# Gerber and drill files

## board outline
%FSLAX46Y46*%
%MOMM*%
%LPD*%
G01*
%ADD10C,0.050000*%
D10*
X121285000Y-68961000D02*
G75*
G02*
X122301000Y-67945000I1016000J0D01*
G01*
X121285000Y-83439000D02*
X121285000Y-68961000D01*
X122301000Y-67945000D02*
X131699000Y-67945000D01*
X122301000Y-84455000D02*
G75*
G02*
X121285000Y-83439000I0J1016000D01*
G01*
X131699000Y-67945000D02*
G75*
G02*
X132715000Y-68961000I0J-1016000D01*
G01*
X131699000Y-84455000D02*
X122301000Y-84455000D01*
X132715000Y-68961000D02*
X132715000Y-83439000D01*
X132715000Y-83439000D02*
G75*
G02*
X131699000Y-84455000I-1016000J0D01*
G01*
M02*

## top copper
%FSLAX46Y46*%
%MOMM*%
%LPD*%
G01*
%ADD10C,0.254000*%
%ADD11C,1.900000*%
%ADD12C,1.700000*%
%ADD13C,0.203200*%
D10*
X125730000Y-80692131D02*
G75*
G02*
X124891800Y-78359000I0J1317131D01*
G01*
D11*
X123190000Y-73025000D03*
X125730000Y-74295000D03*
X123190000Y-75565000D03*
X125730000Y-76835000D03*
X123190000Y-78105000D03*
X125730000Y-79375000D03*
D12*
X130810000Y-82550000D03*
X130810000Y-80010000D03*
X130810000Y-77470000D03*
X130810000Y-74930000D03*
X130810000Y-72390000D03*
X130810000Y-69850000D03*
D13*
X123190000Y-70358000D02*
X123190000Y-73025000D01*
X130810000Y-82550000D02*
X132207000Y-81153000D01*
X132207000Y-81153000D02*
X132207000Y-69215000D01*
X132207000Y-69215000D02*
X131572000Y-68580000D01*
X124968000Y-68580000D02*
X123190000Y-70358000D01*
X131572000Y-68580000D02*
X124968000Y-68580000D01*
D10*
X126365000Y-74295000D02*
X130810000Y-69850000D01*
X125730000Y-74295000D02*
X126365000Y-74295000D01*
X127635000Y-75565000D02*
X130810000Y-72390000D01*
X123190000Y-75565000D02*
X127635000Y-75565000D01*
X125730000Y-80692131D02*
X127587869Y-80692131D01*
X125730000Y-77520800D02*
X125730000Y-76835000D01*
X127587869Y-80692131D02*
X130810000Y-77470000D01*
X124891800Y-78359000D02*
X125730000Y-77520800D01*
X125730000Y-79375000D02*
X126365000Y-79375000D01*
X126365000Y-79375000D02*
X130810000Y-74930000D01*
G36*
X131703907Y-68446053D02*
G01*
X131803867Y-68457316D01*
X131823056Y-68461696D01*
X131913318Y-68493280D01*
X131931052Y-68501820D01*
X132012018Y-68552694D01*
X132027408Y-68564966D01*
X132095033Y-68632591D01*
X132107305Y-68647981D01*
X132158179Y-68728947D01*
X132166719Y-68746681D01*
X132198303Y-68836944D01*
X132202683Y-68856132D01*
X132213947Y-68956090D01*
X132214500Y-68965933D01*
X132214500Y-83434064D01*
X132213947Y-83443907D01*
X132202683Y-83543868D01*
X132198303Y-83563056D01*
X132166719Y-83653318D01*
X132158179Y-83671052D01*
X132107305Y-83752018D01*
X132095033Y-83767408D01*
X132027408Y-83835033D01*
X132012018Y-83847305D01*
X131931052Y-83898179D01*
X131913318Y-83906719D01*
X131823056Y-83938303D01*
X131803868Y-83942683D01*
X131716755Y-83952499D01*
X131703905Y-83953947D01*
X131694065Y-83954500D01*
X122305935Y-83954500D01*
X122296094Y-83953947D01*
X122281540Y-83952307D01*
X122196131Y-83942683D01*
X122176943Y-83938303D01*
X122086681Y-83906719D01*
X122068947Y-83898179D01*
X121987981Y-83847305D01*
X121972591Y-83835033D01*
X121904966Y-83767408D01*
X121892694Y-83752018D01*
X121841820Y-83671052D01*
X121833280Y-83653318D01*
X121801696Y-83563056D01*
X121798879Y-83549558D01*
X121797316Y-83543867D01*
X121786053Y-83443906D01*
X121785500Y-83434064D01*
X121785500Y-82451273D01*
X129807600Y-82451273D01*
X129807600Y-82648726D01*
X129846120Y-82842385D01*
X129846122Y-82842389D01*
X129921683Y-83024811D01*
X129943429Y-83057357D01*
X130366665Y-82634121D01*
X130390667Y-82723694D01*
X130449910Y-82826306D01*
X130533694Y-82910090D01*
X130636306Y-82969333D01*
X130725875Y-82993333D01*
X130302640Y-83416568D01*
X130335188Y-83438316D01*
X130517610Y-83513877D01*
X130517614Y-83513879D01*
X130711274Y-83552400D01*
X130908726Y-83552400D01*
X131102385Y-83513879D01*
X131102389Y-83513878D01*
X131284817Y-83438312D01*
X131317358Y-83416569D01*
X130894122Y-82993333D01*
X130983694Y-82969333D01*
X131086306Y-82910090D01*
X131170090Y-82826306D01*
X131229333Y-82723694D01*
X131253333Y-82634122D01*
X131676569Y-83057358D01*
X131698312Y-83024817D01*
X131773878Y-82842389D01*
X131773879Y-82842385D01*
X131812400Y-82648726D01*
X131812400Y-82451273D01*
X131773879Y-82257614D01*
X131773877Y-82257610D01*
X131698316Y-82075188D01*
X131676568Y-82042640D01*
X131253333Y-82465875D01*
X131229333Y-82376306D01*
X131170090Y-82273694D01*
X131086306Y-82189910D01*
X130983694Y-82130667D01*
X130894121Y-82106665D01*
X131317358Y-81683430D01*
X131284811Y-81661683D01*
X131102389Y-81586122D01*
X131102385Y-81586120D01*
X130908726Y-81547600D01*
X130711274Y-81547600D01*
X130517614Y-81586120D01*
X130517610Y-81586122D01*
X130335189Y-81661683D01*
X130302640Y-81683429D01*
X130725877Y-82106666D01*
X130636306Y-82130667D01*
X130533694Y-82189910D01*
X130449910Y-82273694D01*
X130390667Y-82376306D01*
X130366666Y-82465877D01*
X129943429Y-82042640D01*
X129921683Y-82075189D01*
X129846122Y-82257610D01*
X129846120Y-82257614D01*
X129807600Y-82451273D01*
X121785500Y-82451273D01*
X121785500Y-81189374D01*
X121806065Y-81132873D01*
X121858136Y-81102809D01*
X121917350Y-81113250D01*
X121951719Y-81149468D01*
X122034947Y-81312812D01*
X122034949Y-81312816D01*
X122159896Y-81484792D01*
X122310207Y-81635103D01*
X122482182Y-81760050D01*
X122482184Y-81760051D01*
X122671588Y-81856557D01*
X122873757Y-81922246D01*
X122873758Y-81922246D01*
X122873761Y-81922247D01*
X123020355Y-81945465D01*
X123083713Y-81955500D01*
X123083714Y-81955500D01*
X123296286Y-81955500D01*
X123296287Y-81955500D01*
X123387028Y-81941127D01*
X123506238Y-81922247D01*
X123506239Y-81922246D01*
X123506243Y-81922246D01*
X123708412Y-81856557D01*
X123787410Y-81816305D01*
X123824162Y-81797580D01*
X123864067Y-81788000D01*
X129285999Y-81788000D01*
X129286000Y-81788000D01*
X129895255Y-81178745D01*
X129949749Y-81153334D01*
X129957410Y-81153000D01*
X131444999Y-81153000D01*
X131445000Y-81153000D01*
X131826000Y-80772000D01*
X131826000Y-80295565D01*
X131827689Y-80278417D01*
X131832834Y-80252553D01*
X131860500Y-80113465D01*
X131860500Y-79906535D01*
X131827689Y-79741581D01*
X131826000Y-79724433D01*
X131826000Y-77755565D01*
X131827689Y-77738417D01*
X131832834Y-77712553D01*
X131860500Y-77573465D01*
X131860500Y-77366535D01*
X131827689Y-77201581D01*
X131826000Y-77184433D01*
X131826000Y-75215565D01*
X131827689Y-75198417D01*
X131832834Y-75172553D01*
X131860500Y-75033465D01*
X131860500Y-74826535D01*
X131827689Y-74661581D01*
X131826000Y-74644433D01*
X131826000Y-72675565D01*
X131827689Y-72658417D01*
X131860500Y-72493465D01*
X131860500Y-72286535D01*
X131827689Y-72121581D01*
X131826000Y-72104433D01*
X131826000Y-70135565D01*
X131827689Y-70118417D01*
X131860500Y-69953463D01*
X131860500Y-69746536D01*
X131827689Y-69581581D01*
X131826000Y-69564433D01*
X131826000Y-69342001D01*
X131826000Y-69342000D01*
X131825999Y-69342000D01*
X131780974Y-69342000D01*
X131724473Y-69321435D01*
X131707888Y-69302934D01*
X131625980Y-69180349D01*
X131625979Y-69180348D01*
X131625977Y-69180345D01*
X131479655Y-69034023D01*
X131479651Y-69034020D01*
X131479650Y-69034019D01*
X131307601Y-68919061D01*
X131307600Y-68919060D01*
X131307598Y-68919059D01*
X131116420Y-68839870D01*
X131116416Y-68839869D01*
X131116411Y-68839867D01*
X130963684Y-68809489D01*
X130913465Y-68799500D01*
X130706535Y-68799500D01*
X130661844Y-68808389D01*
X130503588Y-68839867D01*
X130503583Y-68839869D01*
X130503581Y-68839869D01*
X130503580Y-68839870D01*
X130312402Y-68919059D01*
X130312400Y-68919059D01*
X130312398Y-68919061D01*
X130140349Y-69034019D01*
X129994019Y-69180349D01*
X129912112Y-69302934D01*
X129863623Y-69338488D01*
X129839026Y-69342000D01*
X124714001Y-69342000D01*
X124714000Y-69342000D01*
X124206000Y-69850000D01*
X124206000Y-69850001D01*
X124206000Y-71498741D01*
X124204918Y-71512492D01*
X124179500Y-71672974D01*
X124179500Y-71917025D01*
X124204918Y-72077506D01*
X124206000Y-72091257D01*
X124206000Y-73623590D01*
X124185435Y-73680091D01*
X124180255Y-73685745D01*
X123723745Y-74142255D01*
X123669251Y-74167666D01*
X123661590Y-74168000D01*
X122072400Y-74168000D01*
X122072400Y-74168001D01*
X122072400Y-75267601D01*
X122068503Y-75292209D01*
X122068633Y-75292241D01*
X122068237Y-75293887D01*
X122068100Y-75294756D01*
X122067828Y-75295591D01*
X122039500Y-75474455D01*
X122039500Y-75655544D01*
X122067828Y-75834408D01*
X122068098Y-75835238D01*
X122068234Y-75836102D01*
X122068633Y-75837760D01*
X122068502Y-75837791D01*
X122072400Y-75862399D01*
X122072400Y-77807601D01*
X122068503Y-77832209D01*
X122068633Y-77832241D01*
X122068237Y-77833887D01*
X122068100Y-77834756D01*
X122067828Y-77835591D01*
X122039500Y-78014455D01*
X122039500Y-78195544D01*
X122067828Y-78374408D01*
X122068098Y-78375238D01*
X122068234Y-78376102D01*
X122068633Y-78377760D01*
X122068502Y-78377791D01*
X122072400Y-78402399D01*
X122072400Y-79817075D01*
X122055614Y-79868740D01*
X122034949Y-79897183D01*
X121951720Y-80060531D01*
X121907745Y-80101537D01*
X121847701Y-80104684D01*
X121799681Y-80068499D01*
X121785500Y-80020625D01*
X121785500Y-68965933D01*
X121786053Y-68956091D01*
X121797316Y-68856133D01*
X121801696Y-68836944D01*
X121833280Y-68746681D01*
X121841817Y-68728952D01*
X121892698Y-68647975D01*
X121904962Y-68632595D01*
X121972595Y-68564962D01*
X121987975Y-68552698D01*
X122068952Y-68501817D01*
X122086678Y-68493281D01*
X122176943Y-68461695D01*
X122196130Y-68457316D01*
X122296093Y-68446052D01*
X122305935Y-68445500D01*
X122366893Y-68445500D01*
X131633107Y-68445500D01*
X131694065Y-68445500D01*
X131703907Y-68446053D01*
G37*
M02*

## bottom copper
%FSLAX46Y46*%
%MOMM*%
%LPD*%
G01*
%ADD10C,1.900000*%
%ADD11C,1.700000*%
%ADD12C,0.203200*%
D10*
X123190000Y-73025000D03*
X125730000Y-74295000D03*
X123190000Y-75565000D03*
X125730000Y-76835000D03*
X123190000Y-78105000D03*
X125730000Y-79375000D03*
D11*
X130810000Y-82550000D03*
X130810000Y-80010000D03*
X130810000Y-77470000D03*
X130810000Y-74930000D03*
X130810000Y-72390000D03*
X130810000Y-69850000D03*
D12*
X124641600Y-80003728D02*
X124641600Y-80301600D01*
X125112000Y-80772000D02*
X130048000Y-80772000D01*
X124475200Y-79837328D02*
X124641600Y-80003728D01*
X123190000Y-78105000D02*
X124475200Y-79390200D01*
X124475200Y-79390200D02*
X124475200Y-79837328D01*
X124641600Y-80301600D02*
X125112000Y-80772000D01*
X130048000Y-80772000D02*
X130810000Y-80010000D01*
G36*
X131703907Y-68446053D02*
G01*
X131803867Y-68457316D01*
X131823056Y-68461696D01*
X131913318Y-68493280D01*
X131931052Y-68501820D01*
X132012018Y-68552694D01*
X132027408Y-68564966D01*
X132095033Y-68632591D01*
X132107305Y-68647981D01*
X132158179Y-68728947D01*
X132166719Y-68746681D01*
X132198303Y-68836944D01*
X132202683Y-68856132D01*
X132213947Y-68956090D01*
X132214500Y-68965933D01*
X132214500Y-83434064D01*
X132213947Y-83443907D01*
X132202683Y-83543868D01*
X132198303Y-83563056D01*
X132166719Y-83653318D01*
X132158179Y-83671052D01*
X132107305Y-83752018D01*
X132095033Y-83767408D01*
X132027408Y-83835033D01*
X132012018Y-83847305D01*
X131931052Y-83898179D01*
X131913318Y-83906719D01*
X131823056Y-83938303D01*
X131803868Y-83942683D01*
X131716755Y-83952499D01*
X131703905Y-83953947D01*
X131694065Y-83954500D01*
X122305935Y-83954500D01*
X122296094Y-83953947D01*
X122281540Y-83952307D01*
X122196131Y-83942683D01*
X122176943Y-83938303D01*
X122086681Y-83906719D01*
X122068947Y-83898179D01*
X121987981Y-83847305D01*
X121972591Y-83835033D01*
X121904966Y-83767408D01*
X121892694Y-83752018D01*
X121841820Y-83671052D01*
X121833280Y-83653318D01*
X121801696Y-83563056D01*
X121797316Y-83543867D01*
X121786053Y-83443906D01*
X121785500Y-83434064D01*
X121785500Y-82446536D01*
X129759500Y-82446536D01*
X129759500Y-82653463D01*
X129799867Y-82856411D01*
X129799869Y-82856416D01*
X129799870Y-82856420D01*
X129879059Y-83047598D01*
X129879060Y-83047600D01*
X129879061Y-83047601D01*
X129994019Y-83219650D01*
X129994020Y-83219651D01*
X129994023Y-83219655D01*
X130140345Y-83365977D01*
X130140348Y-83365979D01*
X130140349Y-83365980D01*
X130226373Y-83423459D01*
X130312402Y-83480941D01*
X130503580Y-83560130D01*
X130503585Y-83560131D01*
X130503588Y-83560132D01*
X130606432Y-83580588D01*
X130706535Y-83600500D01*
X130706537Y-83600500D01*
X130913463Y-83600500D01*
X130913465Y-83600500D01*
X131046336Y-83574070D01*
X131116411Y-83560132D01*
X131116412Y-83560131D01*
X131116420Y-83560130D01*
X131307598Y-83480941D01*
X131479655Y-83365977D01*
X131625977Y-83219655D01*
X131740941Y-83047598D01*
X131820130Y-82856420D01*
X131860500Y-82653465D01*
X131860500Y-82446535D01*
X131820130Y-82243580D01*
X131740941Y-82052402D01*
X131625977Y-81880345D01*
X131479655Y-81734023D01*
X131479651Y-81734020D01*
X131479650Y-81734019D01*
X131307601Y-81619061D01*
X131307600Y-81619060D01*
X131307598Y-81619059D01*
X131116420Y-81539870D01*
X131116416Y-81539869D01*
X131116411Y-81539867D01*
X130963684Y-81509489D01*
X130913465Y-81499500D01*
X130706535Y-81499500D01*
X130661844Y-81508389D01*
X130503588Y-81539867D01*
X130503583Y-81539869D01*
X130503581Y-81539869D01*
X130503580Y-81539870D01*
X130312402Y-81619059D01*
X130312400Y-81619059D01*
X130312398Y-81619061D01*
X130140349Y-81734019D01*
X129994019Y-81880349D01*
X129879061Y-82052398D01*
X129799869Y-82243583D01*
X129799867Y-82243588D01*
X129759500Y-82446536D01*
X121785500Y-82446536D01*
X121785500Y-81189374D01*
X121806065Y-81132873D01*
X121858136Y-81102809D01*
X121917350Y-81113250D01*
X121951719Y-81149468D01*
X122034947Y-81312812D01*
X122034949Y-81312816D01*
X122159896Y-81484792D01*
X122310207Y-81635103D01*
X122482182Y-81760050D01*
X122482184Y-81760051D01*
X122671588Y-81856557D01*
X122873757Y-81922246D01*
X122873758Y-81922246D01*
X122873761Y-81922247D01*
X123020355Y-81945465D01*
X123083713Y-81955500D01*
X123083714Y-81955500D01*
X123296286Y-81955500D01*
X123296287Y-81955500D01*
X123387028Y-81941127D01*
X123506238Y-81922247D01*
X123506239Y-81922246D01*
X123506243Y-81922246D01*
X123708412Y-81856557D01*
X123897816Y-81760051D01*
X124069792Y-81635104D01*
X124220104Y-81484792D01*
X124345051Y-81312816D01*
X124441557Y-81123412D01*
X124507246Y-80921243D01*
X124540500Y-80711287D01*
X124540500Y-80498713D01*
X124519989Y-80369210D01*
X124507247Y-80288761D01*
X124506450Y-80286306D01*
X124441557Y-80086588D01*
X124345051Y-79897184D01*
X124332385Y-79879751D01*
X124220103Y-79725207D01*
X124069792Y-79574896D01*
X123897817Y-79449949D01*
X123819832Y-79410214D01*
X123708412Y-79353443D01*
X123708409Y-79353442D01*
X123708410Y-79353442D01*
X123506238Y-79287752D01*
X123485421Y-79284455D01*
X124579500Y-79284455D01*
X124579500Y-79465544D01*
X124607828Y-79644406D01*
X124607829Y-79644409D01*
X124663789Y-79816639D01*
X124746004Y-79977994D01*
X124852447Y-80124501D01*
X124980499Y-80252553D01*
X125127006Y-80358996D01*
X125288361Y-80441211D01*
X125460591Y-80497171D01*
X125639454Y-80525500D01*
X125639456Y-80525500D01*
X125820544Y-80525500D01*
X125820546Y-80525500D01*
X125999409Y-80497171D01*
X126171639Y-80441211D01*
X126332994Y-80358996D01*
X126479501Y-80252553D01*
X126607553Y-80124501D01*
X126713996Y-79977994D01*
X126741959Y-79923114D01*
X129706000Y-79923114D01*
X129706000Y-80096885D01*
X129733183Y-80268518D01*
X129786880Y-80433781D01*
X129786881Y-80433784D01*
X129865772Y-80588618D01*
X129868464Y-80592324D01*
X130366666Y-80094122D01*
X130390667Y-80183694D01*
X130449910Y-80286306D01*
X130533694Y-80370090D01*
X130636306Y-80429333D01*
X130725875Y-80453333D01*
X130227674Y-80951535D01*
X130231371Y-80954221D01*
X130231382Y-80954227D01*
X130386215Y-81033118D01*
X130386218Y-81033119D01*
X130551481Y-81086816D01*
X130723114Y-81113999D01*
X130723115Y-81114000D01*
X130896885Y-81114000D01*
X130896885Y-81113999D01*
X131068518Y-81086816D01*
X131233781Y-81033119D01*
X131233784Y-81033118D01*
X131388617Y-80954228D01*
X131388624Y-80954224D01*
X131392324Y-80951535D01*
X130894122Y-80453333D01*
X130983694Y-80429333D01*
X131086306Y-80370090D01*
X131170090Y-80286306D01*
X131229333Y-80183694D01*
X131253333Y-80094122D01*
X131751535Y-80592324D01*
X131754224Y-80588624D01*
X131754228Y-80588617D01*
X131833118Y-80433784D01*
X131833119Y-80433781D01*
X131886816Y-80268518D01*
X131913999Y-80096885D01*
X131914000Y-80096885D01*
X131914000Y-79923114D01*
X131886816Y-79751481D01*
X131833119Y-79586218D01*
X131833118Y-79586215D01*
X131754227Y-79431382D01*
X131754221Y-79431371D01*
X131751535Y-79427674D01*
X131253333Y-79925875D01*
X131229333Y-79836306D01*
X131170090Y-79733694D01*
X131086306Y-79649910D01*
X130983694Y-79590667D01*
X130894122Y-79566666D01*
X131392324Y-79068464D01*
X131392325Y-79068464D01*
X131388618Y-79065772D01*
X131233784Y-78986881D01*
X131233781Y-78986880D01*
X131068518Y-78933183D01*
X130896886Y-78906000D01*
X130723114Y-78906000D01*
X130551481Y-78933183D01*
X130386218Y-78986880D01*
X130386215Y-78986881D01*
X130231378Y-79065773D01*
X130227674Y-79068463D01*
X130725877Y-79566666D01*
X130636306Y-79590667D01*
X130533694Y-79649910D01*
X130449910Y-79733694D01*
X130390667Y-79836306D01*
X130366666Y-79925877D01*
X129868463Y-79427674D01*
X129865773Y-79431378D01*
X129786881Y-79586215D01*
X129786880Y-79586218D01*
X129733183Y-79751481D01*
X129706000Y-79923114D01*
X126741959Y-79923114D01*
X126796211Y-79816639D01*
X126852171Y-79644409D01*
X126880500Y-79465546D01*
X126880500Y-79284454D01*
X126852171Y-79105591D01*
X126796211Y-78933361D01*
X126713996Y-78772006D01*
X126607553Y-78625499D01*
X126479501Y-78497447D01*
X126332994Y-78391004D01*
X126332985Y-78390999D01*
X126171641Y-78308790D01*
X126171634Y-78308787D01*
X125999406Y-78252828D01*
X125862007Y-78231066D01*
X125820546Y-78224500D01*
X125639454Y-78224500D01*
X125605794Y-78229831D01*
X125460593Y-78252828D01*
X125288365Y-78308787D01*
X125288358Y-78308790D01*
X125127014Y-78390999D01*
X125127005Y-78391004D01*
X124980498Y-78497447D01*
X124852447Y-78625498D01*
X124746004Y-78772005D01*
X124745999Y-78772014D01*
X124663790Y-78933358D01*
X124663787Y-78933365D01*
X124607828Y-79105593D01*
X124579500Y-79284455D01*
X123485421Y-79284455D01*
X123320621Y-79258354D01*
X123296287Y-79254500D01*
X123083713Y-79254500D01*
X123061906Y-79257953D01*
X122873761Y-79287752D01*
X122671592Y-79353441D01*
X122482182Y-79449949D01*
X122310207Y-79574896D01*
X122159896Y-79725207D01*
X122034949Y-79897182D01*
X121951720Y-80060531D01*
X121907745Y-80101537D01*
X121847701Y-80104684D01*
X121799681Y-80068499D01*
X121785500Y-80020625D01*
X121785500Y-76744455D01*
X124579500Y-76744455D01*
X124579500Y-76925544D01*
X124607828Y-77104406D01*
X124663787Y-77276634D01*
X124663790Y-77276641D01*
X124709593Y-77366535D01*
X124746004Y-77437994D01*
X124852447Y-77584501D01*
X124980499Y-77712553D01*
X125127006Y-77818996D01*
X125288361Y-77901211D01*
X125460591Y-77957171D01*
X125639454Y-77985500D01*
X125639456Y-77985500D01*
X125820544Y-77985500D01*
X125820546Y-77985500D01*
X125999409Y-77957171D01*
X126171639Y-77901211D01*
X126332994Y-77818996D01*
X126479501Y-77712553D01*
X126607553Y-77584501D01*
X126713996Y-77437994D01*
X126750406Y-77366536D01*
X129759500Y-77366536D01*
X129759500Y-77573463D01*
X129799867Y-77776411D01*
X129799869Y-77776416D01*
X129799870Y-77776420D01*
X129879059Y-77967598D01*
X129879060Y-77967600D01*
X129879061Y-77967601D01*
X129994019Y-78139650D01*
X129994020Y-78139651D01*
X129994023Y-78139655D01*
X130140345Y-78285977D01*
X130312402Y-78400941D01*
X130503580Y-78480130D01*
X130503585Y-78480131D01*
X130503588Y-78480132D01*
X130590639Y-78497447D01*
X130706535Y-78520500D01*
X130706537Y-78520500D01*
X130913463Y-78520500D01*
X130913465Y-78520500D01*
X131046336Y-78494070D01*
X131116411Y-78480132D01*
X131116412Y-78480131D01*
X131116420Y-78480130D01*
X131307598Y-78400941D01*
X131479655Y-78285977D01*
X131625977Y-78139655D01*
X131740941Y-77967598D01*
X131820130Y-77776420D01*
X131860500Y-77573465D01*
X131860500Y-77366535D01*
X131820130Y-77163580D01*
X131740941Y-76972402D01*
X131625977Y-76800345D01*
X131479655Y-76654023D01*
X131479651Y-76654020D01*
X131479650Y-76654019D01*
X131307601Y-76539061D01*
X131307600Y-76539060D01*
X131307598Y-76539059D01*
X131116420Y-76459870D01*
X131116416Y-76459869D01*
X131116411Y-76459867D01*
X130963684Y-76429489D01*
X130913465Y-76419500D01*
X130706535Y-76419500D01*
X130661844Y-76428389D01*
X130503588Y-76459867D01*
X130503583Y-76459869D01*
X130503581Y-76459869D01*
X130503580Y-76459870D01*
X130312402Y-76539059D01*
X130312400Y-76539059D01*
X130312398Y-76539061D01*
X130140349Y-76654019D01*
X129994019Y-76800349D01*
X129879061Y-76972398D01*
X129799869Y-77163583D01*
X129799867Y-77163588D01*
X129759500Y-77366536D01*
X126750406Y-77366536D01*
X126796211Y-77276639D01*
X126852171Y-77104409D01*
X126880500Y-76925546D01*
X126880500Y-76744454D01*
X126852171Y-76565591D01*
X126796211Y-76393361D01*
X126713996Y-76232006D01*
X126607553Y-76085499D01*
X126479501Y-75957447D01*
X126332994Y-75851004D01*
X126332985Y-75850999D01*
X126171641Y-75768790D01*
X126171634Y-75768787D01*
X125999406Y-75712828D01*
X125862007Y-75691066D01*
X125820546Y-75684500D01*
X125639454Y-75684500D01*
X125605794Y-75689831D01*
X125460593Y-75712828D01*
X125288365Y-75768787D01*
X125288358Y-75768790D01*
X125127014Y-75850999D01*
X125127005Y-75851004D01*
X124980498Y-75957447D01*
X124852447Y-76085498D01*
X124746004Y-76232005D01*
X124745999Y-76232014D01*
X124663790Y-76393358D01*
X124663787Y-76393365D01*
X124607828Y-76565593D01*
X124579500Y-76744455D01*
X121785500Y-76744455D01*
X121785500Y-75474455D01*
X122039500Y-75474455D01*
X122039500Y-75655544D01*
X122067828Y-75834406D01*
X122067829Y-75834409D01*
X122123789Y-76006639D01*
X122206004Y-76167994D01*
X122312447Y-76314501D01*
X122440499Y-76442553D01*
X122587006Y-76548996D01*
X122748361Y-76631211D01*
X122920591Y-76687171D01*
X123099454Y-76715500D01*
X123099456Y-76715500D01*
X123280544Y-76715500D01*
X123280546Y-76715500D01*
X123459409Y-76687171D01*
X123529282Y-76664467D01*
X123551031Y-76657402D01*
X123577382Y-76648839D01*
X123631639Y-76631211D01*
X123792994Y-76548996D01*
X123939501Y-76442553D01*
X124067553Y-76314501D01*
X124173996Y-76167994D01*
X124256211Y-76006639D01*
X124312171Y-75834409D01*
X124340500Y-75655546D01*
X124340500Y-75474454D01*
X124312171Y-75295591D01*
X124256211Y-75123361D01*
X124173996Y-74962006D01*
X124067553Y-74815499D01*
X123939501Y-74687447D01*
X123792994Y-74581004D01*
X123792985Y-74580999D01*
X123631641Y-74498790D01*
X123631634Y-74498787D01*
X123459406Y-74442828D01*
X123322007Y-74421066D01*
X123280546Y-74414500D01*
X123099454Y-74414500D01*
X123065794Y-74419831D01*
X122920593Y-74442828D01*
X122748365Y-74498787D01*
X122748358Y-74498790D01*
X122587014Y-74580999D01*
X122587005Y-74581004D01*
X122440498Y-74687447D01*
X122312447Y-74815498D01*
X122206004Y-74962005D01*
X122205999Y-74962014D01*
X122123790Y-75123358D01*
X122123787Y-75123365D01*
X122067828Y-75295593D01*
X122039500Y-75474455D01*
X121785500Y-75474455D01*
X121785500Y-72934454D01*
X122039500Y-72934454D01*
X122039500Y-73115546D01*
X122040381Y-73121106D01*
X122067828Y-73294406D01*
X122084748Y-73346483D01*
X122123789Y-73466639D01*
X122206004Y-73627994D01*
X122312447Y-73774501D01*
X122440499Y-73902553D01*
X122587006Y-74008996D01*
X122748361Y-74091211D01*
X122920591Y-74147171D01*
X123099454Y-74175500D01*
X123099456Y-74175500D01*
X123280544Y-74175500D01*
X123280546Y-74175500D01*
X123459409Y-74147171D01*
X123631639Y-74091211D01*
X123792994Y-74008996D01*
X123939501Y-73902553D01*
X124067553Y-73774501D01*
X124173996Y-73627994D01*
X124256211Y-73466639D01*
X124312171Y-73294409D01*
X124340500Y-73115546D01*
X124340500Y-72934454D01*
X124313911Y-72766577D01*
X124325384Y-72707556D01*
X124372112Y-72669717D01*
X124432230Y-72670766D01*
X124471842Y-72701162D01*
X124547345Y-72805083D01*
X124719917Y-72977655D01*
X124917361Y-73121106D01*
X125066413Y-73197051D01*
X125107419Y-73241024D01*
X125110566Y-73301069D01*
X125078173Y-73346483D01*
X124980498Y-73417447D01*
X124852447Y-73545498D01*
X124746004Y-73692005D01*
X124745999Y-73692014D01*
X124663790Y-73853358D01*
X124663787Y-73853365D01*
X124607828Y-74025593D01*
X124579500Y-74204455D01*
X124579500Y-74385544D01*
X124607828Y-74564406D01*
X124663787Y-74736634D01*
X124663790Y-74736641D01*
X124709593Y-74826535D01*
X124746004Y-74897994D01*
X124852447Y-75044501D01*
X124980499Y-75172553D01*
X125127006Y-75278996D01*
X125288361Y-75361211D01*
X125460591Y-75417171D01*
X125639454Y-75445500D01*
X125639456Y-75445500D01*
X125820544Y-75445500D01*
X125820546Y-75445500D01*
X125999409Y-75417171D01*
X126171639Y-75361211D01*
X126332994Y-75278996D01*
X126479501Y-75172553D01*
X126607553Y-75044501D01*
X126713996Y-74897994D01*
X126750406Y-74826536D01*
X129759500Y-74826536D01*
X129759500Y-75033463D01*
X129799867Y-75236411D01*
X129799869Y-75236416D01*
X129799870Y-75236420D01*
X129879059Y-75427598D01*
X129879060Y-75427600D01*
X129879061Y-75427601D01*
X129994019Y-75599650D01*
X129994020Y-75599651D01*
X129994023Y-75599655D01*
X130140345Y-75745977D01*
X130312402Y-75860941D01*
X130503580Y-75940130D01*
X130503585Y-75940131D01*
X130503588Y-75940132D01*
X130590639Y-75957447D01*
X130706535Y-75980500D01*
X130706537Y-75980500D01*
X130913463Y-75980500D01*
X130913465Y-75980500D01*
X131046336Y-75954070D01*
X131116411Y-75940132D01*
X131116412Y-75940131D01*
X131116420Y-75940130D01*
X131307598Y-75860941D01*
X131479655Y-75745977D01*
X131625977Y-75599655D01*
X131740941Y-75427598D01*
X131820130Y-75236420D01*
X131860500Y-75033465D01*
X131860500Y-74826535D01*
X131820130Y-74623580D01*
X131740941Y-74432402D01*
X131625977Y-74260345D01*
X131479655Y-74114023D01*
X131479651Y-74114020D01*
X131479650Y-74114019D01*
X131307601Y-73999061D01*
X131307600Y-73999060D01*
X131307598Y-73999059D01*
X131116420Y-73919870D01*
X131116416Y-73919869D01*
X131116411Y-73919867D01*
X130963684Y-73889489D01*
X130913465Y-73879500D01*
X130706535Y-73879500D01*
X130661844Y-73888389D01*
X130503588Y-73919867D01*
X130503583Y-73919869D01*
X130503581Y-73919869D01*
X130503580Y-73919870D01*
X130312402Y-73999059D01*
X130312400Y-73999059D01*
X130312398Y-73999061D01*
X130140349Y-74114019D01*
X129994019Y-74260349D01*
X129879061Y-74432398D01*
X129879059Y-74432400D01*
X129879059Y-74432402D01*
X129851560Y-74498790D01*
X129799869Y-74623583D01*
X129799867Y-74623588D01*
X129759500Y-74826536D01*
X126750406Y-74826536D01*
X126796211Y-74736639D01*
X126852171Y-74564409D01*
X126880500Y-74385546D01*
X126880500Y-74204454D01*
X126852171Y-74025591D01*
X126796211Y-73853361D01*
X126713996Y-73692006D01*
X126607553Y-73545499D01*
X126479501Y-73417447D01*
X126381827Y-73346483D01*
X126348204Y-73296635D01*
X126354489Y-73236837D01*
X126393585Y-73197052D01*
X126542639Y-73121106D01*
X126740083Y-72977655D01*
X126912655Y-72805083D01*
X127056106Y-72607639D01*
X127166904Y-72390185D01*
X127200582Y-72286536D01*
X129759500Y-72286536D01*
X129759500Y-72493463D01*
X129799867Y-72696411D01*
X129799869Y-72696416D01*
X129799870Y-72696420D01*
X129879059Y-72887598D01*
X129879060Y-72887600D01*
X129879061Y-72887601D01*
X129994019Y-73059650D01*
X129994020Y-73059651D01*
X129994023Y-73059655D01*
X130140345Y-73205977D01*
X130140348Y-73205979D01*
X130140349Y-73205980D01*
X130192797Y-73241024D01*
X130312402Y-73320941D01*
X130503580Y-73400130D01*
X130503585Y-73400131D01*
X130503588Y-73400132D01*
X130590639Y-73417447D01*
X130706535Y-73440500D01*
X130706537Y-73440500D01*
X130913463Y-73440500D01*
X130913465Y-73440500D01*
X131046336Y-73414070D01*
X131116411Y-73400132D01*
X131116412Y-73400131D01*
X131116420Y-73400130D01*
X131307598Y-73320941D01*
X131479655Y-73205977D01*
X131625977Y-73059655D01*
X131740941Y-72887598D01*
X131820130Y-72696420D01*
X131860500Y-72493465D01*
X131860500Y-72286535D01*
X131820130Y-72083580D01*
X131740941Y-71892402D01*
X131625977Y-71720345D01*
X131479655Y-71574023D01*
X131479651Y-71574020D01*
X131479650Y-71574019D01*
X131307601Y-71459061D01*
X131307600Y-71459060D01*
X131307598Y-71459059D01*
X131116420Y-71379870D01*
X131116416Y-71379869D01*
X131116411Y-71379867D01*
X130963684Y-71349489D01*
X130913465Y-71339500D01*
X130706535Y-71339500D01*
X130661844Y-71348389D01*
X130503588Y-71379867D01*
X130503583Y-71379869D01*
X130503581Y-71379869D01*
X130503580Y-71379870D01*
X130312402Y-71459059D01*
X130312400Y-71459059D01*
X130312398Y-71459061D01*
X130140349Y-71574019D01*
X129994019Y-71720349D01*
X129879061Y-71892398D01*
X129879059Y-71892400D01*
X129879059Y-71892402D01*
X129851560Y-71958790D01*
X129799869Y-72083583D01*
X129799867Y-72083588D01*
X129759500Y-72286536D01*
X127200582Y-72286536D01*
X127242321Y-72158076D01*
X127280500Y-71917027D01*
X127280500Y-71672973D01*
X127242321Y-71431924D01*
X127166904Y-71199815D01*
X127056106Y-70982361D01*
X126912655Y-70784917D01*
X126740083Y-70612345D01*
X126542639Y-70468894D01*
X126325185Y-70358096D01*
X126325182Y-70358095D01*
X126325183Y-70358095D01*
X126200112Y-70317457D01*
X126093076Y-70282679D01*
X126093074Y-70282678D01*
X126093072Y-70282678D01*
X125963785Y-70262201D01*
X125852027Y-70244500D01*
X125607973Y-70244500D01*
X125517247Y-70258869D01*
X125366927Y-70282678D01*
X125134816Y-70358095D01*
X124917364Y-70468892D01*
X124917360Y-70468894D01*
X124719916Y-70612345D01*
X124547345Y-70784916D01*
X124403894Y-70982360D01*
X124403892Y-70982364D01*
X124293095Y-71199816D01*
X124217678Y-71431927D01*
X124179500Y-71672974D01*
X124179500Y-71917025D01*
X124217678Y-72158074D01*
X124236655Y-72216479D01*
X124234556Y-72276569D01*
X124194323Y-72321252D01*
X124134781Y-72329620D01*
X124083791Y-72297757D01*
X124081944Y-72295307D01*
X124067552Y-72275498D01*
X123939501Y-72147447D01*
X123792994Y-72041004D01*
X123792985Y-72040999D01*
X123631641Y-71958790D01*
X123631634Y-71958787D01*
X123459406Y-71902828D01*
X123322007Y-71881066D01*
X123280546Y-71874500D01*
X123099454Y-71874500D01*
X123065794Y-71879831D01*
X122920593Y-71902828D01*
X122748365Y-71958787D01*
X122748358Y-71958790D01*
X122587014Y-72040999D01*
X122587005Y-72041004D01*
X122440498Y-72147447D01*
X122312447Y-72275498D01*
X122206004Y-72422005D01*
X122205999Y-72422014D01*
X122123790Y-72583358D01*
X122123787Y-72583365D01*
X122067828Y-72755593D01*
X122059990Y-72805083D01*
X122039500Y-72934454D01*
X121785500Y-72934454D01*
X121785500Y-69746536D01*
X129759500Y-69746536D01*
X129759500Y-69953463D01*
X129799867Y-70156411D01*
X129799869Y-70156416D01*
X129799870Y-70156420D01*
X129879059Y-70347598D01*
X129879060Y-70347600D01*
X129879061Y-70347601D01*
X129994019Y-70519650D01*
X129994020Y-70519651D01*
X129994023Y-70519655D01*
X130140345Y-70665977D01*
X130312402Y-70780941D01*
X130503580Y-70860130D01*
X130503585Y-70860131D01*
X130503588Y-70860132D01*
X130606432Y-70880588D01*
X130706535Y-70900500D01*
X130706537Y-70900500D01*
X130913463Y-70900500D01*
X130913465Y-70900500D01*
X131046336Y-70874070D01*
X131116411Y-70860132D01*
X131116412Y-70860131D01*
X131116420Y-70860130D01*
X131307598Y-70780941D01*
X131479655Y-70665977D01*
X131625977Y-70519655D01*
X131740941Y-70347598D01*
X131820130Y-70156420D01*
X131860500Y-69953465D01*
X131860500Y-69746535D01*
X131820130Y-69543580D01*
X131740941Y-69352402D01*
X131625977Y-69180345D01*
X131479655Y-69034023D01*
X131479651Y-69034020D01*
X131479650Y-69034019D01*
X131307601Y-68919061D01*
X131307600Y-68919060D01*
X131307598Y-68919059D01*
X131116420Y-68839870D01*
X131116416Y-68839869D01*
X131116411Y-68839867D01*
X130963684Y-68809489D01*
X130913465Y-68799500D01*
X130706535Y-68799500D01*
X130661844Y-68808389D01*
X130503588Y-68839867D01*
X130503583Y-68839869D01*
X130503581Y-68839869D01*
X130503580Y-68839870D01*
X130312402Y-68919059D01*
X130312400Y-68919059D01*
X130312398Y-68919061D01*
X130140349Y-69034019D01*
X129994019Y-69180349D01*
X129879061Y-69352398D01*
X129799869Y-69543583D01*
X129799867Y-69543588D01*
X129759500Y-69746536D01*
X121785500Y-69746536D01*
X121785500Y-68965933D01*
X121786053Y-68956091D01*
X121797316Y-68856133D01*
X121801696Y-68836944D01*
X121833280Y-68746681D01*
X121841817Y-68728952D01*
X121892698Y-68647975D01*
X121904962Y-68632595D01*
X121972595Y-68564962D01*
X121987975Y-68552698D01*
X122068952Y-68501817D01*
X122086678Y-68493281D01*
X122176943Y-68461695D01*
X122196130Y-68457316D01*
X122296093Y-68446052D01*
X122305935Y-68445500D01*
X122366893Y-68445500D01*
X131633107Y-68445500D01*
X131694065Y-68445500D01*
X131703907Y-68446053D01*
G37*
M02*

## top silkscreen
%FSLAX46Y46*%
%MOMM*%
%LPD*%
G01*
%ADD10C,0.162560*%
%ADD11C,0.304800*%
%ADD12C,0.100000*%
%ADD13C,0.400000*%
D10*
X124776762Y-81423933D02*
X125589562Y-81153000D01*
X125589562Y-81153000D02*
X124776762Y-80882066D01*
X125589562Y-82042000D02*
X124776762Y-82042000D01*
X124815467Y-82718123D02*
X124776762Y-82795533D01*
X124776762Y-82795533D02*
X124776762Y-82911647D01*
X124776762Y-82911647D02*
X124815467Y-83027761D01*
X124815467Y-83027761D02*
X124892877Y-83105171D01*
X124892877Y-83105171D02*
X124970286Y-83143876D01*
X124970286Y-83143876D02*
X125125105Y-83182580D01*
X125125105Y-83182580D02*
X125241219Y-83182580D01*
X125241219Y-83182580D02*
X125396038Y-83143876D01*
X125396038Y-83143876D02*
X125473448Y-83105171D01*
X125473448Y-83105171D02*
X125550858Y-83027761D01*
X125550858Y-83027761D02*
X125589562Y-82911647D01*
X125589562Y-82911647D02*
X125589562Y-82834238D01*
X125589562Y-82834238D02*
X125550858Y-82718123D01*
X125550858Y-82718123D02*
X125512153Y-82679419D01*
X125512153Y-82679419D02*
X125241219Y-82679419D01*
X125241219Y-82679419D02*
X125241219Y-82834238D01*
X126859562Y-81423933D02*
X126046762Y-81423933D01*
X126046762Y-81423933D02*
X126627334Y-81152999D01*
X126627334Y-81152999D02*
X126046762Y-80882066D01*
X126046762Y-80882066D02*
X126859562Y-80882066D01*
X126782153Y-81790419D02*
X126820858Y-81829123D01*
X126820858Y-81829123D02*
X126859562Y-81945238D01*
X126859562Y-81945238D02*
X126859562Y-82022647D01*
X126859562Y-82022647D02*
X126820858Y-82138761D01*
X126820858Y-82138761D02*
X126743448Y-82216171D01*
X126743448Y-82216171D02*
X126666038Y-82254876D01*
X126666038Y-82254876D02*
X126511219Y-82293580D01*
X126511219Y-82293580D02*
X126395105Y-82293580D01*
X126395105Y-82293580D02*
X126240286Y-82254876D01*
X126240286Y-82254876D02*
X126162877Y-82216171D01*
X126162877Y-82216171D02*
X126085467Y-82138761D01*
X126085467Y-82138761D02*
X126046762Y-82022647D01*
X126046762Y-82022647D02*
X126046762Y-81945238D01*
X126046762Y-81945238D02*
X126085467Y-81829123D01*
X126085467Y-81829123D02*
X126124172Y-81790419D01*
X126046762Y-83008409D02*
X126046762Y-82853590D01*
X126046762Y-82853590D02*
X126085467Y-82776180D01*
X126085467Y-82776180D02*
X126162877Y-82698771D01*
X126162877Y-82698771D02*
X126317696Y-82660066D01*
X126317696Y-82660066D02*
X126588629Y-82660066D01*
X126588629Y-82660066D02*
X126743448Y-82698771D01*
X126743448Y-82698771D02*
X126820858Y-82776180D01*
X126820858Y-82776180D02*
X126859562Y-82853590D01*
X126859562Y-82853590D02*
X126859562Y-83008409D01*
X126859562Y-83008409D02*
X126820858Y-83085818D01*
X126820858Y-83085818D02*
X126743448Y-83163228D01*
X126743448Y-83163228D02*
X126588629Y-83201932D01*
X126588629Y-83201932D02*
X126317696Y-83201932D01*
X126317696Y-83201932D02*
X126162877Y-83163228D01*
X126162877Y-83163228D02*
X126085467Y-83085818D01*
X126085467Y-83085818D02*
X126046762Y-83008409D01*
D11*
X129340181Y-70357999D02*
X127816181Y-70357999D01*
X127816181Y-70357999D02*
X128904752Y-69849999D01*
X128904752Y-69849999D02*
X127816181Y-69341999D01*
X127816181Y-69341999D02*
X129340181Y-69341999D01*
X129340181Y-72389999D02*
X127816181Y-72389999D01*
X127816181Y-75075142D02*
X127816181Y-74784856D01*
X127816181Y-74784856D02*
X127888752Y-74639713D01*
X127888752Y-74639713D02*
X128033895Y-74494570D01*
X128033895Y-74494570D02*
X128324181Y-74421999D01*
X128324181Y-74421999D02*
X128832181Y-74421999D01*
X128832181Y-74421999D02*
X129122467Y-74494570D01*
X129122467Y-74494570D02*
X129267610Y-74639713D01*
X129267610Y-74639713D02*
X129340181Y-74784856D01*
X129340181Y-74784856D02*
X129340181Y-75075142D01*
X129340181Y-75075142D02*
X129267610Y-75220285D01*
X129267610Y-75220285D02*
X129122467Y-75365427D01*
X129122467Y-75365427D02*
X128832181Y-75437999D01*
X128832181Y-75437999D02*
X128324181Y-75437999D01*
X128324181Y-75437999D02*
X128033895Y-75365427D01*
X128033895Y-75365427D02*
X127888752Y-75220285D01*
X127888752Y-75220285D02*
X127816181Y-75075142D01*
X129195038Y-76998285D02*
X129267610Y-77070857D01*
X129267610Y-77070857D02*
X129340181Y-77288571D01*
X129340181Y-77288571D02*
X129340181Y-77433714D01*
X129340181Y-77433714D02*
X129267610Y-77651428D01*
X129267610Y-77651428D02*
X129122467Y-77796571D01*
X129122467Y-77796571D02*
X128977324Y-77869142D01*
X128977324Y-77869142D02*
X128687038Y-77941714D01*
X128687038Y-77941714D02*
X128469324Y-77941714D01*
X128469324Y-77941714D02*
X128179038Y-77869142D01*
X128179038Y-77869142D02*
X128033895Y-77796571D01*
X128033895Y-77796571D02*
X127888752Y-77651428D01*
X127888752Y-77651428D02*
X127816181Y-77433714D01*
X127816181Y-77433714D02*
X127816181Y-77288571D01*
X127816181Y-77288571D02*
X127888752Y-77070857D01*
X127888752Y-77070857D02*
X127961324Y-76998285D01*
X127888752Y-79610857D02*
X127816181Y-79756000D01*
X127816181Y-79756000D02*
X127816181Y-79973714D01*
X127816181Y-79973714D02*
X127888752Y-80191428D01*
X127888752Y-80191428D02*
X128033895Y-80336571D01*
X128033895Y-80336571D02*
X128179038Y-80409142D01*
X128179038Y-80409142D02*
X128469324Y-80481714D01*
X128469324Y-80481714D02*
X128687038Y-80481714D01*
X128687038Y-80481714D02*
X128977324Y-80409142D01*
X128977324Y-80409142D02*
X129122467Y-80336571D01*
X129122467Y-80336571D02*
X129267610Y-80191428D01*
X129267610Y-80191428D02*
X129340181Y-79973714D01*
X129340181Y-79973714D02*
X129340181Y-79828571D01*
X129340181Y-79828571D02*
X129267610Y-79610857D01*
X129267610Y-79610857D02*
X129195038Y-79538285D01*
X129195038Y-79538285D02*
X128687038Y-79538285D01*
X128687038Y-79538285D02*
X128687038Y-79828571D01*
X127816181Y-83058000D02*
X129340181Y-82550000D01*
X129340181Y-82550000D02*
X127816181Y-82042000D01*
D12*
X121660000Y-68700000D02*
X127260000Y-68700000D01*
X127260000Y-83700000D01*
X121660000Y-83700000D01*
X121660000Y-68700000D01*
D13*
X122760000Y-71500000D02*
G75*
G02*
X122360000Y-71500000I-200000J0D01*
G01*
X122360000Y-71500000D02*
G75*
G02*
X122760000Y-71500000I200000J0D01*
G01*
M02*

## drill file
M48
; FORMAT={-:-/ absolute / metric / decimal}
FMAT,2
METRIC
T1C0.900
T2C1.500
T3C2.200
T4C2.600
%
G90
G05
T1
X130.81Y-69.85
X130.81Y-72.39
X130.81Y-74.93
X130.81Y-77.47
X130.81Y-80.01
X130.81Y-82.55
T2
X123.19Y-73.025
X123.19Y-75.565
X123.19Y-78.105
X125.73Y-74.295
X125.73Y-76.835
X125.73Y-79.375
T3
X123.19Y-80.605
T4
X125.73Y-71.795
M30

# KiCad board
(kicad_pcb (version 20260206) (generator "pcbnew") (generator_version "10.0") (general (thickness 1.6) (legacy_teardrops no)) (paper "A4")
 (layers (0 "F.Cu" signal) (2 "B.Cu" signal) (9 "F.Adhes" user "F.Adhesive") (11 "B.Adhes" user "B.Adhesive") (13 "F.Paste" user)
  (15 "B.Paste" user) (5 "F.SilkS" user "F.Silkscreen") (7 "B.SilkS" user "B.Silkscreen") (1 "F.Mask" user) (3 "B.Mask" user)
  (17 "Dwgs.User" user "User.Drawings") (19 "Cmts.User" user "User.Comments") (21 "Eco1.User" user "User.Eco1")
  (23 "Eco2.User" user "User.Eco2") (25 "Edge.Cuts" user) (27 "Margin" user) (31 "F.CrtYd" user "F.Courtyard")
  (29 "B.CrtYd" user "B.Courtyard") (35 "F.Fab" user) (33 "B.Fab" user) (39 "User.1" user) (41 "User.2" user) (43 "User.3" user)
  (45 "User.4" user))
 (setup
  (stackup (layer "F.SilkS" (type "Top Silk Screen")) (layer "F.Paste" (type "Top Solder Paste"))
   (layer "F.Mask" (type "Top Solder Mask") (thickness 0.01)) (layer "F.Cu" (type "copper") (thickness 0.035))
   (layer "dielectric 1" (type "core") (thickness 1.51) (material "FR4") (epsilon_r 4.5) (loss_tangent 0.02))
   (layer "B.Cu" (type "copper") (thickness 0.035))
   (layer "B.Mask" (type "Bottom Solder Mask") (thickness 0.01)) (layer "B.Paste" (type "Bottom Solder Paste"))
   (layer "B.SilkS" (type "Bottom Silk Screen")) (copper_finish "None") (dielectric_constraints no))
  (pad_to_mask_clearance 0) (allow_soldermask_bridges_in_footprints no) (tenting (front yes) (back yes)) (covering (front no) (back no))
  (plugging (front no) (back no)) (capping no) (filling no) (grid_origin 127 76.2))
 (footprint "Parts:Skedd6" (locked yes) (layer "F.Cu") (at 124.46 76.2)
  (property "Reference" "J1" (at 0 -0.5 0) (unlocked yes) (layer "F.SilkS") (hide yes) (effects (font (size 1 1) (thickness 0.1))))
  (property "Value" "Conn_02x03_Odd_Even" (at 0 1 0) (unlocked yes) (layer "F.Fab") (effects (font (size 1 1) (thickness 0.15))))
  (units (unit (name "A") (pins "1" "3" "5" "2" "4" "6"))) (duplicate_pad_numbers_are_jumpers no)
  (fp_rect (start -2.8 -7.5) (end 2.8 7.5) (stroke (width 0.1) (type default)) (fill no) (layer "F.SilkS"))
  (fp_circle (center -1.9 -4.7) (end -1.9 -4.3) (stroke (width 0) (type default)) (fill yes) (layer "F.SilkS"))
  (pad "" np_thru_hole circle (at -1.27 4.405) (size 2.2 2.2) (drill 2.2) (layers "F.Cu" "F.Mask" "F.Paste"))
  (pad "" np_thru_hole circle (at 1.27 -4.405) (size 2.6 2.6) (drill 2.6) (layers "F.Cu" "F.Mask" "F.Paste"))
  (pad "1" thru_hole circle (at -1.27 -3.175) (size 1.9 1.9) (drill 1.5) (layers "*.Cu" "F.Mask" "F.Paste") (remove_unused_layers no)
   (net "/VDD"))
  (pad "2" thru_hole circle (at 1.27 -1.905) (size 1.9 1.9) (drill 1.5) (layers "*.Cu" "F.Mask" "F.Paste") (remove_unused_layers no)
   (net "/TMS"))
  (pad "3" thru_hole circle (at -1.27 -0.635) (size 1.9 1.9) (drill 1.5) (layers "*.Cu" "F.Mask" "F.Paste") (remove_unused_layers no)
   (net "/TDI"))
  (pad "4" thru_hole circle (at 1.27 0.635) (size 1.9 1.9) (drill 1.5) (layers "*.Cu" "F.Mask" "F.Paste") (remove_unused_layers no)
   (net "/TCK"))
  (pad "5" thru_hole circle (at -1.27 1.905) (size 1.9 1.9) (drill 1.5) (layers "*.Cu" "F.Mask" "F.Paste") (remove_unused_layers no)
   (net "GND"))
  (pad "6" thru_hole circle (at 1.27 3.175) (size 1.9 1.9) (drill 1.5) (layers "*.Cu" "F.Mask" "F.Paste") (remove_unused_layers no)
   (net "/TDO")))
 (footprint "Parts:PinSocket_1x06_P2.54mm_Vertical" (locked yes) (layer "B.Cu") (at 130.81 82.55)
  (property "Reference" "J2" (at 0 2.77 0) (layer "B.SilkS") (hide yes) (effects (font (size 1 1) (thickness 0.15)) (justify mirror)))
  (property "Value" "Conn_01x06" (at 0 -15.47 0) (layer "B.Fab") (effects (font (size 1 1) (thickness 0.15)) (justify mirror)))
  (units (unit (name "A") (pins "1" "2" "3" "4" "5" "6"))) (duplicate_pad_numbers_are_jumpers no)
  (pad "1" thru_hole circle (at 0 0) (size 1.7 1.7) (drill 0.9) (layers "*.Cu" "*.Mask") (remove_unused_layers no) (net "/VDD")
   (zone_connect 1))
  (pad "2" thru_hole circle (at 0 -2.54) (size 1.7 1.7) (drill 0.9) (layers "*.Cu" "*.Mask") (remove_unused_layers no) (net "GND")
   (zone_connect 1))
  (pad "3" thru_hole circle (at 0 -5.08) (size 1.7 1.7) (drill 0.9) (layers "*.Cu" "*.Mask") (remove_unused_layers no) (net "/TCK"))
  (pad "4" thru_hole circle (at 0 -7.62) (size 1.7 1.7) (drill 0.9) (layers "*.Cu" "*.Mask") (remove_unused_layers no) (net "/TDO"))
  (pad "5" thru_hole circle (at 0 -10.16) (size 1.7 1.7) (drill 0.9) (layers "*.Cu" "*.Mask") (remove_unused_layers no) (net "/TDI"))
  (pad "6" thru_hole circle (at 0 -12.7) (size 1.7 1.7) (drill 0.9) (layers "*.Cu" "*.Mask") (remove_unused_layers no) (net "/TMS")))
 (gr_arc (start 125.73 80.692131) (mid 124.490436 79.820325) (end 124.8918 78.359) (stroke (width 0.254) (type default)) (layer "F.Cu")
  (net "/TCK"))
 (gr_arc (start 121.285 68.961) (mid 121.58258 68.24258) (end 122.301 67.945) (stroke (width 0.05) (type default)) (layer "Edge.Cuts"))
 (gr_line (start 121.285 83.439) (end 121.285 68.961) (stroke (width 0.05) (type default)) (layer "Edge.Cuts"))
 (gr_line (start 122.301 67.945) (end 131.699 67.945) (stroke (width 0.05) (type default)) (layer "Edge.Cuts"))
 (gr_arc (start 122.301 84.455) (mid 121.58258 84.15742) (end 121.285 83.439) (stroke (width 0.05) (type default)) (layer "Edge.Cuts"))
 (gr_arc (start 131.699 67.945) (mid 132.41742 68.24258) (end 132.715 68.961) (stroke (width 0.05) (type default)) (layer "Edge.Cuts"))
 (gr_line (start 131.699 84.455) (end 122.301 84.455) (stroke (width 0.05) (type default)) (layer "Edge.Cuts"))
 (gr_line (start 132.715 68.961) (end 132.715 83.439) (stroke (width 0.05) (type default)) (layer "Edge.Cuts"))
 (gr_arc (start 132.715 83.439) (mid 132.41742 84.15742) (end 131.699 84.455) (stroke (width 0.05) (type default)) (layer "Edge.Cuts"))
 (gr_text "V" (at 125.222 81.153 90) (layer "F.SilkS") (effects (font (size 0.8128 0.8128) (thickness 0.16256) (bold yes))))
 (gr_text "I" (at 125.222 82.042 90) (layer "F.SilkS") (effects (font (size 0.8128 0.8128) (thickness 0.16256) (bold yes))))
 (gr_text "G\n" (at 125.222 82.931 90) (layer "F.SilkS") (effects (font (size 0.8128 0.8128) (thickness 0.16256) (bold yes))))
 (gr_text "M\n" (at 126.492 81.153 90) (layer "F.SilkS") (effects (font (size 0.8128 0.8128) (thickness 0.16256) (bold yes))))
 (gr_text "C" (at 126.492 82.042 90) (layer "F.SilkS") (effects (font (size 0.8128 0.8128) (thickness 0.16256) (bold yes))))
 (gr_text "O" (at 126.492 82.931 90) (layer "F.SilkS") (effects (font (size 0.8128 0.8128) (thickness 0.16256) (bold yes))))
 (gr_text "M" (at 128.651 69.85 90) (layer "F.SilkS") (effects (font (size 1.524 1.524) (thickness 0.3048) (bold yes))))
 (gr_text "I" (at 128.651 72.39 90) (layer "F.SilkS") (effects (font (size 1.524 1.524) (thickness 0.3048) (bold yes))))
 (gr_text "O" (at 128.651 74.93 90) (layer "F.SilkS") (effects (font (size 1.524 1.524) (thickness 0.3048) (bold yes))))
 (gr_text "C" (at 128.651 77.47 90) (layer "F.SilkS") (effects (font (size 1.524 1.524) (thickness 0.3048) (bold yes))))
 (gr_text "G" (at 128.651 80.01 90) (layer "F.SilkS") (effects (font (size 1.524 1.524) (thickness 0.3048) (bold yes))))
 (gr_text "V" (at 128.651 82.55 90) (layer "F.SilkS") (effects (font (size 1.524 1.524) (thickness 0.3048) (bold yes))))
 (segment (start 123.19 70.358) (end 123.19 73.025) (width 0.2032) (layer "F.Cu") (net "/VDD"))
 (segment (start 130.81 82.55) (end 132.207 81.153) (width 0.2032) (layer "F.Cu") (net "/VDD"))
 (segment (start 132.207 81.153) (end 132.207 69.215) (width 0.2032) (layer "F.Cu") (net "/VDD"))
 (segment (start 132.207 69.215) (end 131.572 68.58) (width 0.2032) (layer "F.Cu") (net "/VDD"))
 (segment (start 124.968 68.58) (end 123.19 70.358) (width 0.2032) (layer "F.Cu") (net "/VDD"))
 (segment (start 131.572 68.58) (end 124.968 68.58) (width 0.2032) (layer "F.Cu") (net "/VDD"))
 (segment (start 126.365 74.295) (end 130.81 69.85) (width 0.254) (layer "F.Cu") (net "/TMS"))
 (segment (start 125.73 74.295) (end 126.365 74.295) (width 0.254) (layer "F.Cu") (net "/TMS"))
 (segment (start 127.635 75.565) (end 130.81 72.39) (width 0.254) (layer "F.Cu") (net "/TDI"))
 (segment (start 123.19 75.565) (end 127.635 75.565) (width 0.254) (layer "F.Cu") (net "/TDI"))
 (segment (start 125.73 80.692131) (end 127.587869 80.692131) (width 0.254) (layer "F.Cu") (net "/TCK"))
 (segment (start 125.73 77.5208) (end 125.73 76.835) (width 0.254) (layer "F.Cu") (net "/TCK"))
 (segment (start 127.587869 80.692131) (end 130.81 77.47) (width 0.254) (layer "F.Cu") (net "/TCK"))
 (segment (start 124.8918 78.359) (end 125.73 77.5208) (width 0.254) (layer "F.Cu") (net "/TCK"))
 (segment (start 124.6416 80.003728) (end 124.6416 80.3016) (width 0.2032) (layer "B.Cu") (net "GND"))
 (segment (start 125.112 80.772) (end 130.048 80.772) (width 0.2032) (layer "B.Cu") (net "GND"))
 (segment (start 124.4752 79.837328) (end 124.6416 80.003728) (width 0.2032) (layer "B.Cu") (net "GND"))
 (segment (start 123.19 78.105) (end 124.4752 79.3902) (width 0.2032) (layer "B.Cu") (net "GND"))
 (segment (start 124.4752 79.3902) (end 124.4752 79.837328) (width 0.2032) (layer "B.Cu") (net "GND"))
 (segment (start 124.6416 80.3016) (end 125.112 80.772) (width 0.2032) (layer "B.Cu") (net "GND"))
 (segment (start 130.048 80.772) (end 130.81 80.01) (width 0.2032) (layer "B.Cu") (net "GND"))
 (segment (start 125.73 79.375) (end 126.365 79.375) (width 0.254) (layer "F.Cu") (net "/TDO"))
 (segment (start 126.365 79.375) (end 130.81 74.93) (width 0.254) (layer "F.Cu") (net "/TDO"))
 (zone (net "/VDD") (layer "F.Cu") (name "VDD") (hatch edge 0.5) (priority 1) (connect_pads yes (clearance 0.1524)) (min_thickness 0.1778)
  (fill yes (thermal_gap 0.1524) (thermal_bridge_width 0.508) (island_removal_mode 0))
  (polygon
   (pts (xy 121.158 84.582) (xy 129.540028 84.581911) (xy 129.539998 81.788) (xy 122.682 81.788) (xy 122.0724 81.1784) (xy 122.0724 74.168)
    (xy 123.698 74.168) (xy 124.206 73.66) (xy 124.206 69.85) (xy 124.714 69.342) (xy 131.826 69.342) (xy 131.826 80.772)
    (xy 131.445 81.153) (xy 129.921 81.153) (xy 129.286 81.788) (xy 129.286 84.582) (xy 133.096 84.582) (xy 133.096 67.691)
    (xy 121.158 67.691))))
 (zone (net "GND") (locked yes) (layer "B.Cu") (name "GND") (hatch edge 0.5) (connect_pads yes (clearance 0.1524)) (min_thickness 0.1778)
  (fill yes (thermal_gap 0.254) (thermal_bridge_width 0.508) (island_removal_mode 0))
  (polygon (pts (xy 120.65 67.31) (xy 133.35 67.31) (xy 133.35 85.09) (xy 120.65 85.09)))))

